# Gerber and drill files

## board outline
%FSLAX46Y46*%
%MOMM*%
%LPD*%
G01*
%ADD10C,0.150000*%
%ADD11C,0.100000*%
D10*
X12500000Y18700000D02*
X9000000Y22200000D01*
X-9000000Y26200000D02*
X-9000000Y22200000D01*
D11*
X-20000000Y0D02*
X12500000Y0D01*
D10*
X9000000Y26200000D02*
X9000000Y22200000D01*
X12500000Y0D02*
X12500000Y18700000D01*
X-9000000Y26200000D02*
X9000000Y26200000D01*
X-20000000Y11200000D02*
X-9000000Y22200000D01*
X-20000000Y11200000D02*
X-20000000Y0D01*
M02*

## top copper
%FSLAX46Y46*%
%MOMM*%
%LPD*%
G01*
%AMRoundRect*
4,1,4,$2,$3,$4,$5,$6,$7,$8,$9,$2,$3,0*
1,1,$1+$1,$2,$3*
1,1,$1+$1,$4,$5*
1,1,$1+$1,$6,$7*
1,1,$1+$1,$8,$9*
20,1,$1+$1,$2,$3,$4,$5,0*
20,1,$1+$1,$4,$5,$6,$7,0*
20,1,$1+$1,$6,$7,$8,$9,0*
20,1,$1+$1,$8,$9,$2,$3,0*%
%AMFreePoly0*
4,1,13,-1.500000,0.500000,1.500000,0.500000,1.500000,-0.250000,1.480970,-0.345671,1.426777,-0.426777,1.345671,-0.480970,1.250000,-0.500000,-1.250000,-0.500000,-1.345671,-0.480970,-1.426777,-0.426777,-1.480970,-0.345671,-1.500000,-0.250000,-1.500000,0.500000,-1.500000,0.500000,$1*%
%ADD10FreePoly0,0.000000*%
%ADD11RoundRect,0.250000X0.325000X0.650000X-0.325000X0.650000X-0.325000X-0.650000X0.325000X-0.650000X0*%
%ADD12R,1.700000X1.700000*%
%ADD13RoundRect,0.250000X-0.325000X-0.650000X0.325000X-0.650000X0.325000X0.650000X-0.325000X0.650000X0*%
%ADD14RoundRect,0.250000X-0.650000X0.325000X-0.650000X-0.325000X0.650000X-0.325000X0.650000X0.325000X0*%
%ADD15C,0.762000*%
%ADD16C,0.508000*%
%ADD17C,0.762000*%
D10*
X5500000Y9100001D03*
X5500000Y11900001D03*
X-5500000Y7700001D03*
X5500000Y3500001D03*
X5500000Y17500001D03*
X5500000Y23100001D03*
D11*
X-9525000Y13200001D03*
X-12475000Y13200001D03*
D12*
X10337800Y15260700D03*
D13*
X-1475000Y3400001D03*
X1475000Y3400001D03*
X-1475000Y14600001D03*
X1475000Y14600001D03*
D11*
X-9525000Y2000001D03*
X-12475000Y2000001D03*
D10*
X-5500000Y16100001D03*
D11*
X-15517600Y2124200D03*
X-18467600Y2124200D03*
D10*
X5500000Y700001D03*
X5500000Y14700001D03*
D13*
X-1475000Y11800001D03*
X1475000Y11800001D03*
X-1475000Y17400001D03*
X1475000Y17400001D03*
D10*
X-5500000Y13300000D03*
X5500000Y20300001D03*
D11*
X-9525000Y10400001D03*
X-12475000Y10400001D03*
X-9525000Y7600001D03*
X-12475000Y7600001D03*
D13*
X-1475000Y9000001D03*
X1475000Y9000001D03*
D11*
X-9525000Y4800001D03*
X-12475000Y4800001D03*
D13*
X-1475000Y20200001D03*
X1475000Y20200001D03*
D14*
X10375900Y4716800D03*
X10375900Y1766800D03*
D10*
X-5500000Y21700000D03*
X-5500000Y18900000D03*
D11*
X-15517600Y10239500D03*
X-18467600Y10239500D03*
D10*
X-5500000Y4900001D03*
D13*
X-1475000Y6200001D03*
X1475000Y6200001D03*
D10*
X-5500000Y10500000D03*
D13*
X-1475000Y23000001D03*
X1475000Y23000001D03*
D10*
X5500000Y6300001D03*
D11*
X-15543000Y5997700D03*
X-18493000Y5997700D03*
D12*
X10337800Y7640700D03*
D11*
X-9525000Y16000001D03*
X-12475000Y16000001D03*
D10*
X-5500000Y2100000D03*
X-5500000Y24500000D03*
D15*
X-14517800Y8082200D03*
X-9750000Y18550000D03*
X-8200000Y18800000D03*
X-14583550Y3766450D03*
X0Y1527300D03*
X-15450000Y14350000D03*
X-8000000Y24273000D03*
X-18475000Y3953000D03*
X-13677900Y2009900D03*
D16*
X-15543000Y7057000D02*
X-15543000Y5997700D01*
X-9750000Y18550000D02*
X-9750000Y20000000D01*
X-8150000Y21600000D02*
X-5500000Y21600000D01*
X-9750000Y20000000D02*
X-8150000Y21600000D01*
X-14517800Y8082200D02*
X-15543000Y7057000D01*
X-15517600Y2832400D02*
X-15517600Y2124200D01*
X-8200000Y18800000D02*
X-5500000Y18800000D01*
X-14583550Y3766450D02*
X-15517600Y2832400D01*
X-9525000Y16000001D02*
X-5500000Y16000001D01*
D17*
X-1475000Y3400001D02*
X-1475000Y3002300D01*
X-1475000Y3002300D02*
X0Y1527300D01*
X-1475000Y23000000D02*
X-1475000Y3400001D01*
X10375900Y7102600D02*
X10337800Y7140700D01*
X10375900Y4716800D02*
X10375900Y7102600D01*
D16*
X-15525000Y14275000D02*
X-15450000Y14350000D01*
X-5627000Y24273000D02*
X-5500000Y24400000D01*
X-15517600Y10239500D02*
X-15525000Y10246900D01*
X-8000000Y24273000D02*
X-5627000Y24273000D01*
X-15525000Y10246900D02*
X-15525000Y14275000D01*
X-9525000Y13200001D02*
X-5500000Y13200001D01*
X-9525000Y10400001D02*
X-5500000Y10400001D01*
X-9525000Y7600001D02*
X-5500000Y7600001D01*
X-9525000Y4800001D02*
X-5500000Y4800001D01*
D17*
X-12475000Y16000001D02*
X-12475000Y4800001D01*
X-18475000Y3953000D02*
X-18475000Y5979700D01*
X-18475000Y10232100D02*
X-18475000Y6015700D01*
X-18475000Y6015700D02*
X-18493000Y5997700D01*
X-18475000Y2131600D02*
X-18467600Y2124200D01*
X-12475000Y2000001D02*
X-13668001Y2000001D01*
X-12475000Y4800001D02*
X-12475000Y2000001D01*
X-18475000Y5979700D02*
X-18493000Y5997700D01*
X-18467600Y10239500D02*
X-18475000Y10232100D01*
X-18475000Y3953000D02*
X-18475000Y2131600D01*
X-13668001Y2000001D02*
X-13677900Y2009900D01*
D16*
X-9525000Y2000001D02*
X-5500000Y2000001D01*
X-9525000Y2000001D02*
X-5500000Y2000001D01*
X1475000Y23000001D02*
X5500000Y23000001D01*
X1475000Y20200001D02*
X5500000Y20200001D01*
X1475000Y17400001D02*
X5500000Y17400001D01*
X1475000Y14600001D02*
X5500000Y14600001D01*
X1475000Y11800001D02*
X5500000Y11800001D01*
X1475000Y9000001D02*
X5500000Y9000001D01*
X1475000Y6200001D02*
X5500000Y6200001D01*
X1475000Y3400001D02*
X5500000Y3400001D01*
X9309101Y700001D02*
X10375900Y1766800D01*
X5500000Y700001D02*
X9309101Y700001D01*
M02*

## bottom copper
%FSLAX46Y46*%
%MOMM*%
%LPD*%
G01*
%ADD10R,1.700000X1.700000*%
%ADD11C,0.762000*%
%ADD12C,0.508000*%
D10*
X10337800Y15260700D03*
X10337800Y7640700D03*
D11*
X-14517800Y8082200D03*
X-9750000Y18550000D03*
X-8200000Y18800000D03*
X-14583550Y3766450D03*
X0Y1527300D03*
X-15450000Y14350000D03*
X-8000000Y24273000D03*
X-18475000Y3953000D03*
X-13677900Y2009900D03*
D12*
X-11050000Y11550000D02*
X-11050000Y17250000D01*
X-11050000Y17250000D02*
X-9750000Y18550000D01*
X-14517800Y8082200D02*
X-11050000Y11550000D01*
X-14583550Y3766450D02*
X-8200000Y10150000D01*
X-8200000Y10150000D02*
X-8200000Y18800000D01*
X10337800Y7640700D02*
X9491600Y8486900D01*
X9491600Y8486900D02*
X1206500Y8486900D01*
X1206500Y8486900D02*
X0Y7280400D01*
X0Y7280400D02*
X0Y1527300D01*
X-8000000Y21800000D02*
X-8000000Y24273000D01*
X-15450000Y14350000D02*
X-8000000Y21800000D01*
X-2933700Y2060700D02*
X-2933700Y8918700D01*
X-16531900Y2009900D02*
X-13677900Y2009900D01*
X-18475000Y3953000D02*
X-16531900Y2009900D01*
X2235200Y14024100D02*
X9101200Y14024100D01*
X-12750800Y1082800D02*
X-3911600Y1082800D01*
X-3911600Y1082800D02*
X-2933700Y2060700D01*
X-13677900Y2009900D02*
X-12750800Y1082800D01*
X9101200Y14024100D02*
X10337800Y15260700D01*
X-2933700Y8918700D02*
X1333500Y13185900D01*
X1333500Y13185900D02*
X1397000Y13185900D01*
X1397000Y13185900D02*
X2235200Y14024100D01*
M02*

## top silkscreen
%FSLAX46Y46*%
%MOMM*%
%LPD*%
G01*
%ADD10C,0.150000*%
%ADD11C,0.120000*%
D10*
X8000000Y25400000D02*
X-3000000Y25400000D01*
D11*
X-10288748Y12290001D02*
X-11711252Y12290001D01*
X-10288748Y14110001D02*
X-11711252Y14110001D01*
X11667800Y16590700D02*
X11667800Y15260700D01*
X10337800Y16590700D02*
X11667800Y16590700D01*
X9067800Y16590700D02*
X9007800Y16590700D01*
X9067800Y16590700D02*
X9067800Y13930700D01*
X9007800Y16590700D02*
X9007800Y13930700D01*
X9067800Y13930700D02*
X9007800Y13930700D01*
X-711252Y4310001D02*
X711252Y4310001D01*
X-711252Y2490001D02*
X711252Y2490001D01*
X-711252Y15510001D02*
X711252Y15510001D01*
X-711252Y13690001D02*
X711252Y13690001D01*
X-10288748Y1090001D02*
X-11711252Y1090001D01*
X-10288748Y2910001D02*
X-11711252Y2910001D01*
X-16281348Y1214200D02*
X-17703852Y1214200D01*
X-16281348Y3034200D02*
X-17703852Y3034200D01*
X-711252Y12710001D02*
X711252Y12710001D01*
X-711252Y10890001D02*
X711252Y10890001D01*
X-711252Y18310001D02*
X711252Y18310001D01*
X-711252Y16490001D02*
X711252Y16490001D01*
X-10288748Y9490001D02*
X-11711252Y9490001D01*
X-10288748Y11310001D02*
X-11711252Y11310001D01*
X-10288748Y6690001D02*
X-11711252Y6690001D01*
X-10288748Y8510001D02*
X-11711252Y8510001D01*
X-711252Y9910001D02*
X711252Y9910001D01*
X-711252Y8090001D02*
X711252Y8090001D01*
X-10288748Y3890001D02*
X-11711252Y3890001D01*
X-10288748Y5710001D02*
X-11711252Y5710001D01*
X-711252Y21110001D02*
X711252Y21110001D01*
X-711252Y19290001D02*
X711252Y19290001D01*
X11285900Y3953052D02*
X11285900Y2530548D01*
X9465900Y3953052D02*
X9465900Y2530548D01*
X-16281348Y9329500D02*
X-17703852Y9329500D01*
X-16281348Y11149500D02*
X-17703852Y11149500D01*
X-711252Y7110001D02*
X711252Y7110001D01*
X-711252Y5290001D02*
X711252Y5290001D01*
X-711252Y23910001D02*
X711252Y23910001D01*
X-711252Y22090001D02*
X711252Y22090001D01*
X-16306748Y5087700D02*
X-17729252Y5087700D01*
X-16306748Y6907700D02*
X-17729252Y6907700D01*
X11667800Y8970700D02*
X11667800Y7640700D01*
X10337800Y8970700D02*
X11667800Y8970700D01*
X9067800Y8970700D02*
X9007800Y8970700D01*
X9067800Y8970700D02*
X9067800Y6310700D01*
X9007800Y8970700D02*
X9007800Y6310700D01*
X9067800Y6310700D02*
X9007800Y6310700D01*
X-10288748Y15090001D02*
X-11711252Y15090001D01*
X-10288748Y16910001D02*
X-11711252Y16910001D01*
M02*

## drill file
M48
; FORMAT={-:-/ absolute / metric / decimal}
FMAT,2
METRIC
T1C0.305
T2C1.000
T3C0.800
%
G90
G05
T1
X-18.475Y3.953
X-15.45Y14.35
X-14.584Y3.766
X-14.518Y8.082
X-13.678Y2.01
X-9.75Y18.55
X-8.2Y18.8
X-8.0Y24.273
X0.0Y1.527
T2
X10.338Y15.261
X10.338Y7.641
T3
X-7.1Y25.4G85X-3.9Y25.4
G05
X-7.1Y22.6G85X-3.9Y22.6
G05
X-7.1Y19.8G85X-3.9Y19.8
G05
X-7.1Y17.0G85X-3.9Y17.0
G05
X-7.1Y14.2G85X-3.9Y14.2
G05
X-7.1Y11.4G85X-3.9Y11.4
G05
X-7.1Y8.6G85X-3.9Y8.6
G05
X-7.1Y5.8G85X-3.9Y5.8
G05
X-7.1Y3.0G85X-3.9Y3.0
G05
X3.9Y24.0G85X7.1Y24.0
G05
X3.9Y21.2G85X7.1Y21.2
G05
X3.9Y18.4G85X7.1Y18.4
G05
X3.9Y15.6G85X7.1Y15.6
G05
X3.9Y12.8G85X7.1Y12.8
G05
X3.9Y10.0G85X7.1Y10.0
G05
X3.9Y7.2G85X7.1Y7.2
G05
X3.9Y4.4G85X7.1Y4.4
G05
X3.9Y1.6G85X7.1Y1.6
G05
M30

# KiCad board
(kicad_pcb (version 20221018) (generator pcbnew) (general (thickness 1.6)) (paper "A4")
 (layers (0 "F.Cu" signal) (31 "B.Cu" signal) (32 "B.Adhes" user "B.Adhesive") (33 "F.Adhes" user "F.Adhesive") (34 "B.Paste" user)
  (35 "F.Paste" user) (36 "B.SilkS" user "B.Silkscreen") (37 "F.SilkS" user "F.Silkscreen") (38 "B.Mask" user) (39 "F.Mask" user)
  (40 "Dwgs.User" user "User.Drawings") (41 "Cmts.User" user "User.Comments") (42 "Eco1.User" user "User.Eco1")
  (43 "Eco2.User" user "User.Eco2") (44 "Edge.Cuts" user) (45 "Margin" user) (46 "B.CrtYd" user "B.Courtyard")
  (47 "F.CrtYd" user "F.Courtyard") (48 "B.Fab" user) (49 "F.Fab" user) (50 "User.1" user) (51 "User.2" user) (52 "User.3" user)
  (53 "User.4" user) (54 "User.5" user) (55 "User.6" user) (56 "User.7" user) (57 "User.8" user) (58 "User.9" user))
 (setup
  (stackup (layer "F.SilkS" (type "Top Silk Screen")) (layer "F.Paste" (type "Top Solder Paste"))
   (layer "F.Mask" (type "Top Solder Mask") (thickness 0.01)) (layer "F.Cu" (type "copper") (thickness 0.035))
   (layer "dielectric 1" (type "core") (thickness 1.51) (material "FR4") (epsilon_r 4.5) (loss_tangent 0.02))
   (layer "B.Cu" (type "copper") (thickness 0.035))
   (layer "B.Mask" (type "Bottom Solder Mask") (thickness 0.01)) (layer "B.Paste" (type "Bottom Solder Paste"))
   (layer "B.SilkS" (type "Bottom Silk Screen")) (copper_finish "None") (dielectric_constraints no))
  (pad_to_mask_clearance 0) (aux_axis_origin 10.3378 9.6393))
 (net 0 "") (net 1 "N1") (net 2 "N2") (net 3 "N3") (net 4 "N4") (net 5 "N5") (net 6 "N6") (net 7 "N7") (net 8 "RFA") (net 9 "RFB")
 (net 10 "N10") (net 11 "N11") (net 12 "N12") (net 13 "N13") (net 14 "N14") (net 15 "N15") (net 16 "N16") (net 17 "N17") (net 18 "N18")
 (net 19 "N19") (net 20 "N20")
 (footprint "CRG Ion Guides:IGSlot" (layer "F.Cu") (at 5.5 -10.000001)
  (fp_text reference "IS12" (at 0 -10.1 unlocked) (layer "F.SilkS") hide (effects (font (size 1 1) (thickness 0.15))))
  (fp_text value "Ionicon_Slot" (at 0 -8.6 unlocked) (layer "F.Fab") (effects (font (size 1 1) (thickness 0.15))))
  (pad "" np_thru_hole oval (at 0 0) (size 4 0.8) (drill oval 4 0.8) (layers "*.Mask"))
  (pad "1" smd roundrect (at 0 0.9) (size 3 1) (layers "F.Cu" "F.Mask") (roundrect_rratio 0.25) (chamfer_ratio 0)
   (chamfer top_left top_right) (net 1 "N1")))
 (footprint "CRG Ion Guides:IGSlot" (layer "F.Cu") (at 5.5 -12.800001)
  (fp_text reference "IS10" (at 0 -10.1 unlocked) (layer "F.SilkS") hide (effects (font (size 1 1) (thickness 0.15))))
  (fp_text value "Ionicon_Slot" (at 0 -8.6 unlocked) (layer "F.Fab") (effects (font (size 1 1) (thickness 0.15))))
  (pad "" np_thru_hole oval (at 0 0) (size 4 0.8) (drill oval 4 0.8) (layers "*.Mask"))
  (pad "1" smd roundrect (at 0 0.9) (size 3 1) (layers "F.Cu" "F.Mask") (roundrect_rratio 0.25) (chamfer_ratio 0)
   (chamfer top_left top_right) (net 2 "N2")))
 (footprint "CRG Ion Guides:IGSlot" (layer "F.Cu") (at -5.5 -8.600001)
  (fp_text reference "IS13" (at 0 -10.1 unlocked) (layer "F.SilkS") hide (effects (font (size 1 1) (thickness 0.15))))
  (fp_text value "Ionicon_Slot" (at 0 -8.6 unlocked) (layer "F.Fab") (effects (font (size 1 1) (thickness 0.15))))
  (pad "" np_thru_hole oval (at 0 0) (size 4 0.8) (drill oval 4 0.8) (layers "*.Mask"))
  (pad "1" smd roundrect (at 0 0.9) (size 3 1) (layers "F.Cu" "F.Mask") (roundrect_rratio 0.25) (chamfer_ratio 0)
   (chamfer top_left top_right) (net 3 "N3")))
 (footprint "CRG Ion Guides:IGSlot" (layer "F.Cu") (at 5.5 -4.400001)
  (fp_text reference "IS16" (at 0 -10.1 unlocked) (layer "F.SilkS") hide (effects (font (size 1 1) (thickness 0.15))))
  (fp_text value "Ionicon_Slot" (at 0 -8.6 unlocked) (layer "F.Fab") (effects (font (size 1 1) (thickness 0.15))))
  (pad "" np_thru_hole oval (at 0 0) (size 4 0.8) (drill oval 4 0.8) (layers "*.Mask"))
  (pad "1" smd roundrect (at 0 0.9) (size 3 1) (layers "F.Cu" "F.Mask") (roundrect_rratio 0.25) (chamfer_ratio 0)
   (chamfer top_left top_right) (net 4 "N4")))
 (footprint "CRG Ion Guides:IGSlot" (layer "F.Cu") (at 5.5 -18.400001)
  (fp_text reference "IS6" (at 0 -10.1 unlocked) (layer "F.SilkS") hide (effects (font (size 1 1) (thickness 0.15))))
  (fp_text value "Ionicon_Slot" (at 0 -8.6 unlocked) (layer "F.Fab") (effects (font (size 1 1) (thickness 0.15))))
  (pad "" np_thru_hole oval (at 0 0) (size 4 0.8) (drill oval 4 0.8) (layers "*.Mask"))
  (pad "1" smd roundrect (at 0 0.9) (size 3 1) (layers "F.Cu" "F.Mask") (roundrect_rratio 0.25) (chamfer_ratio 0)
   (chamfer top_left top_right) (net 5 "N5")))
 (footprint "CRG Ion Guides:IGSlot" (layer "F.Cu") (at 5.5 -24.000001)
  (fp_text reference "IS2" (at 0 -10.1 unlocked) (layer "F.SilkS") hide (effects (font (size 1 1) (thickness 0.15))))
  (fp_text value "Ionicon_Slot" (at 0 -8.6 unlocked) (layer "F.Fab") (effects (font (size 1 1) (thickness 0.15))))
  (pad "" np_thru_hole oval (at 0 0) (size 4 0.8) (drill oval 4 0.8) (layers "*.Mask"))
  (pad "1" smd roundrect (at 0 0.9) (size 3 1) (layers "F.Cu" "F.Mask") (roundrect_rratio 0.25) (chamfer_ratio 0)
   (chamfer top_left top_right) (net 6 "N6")))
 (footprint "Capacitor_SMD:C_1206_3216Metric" (layer "F.Cu") (at -11 -13.200001 180)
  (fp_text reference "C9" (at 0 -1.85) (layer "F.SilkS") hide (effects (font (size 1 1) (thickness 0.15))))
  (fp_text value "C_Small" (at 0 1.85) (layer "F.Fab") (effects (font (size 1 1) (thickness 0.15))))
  (fp_line (start -0.711252 -0.91) (end 0.711252 -0.91) (stroke (width 0.12) (type solid)) (layer "F.SilkS"))
  (fp_line (start -0.711252 0.91) (end 0.711252 0.91) (stroke (width 0.12) (type solid)) (layer "F.SilkS"))
  (pad "1" smd roundrect (at -1.475 0 180) (size 1.15 1.8) (layers "F.Cu" "F.Paste" "F.Mask") (roundrect_rratio 0.2173913043) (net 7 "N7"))
  (pad "2" smd roundrect (at 1.475 0 180) (size 1.15 1.8) (layers "F.Cu" "F.Paste" "F.Mask") (roundrect_rratio 0.2173913043) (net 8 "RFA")))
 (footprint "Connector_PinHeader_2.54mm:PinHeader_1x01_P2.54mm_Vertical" (layer "F.Cu") (at 10.3378 -15.2607 -90)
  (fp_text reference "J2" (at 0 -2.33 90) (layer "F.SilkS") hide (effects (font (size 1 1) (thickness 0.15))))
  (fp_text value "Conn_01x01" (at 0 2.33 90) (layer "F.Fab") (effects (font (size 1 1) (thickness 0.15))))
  (fp_line (start -1.33 -1.33) (end 0 -1.33) (stroke (width 0.12) (type solid)) (layer "F.SilkS"))
  (fp_line (start -1.33 0) (end -1.33 -1.33) (stroke (width 0.12) (type solid)) (layer "F.SilkS"))
  (fp_line (start -1.33 1.27) (end -1.33 1.33) (stroke (width 0.12) (type solid)) (layer "F.SilkS"))
  (fp_line (start -1.33 1.27) (end 1.33 1.27) (stroke (width 0.12) (type solid)) (layer "F.SilkS"))
  (fp_line (start -1.33 1.33) (end 1.33 1.33) (stroke (width 0.12) (type solid)) (layer "F.SilkS"))
  (fp_line (start 1.33 1.27) (end 1.33 1.33) (stroke (width 0.12) (type solid)) (layer "F.SilkS"))
  (pad "1" thru_hole rect (at 0 0 270) (size 1.7 1.7) (drill 1) (layers "*.Cu" "*.Mask") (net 8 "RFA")))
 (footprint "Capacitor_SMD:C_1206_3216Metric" (layer "F.Cu") (at 0 -3.400001)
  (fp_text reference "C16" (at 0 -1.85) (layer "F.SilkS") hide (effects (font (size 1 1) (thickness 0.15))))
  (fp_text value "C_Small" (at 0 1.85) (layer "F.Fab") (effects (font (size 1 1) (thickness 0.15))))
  (fp_line (start -0.711252 -0.91) (end 0.711252 -0.91) (stroke (width 0.12) (type solid)) (layer "F.SilkS"))
  (fp_line (start -0.711252 0.91) (end 0.711252 0.91) (stroke (width 0.12) (type solid)) (layer "F.SilkS"))
  (pad "1" smd roundrect (at -1.475 0) (size 1.15 1.8) (layers "F.Cu" "F.Paste" "F.Mask") (roundrect_rratio 0.2173913043) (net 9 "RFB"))
  (pad "2" smd roundrect (at 1.475 0) (size 1.15 1.8) (layers "F.Cu" "F.Paste" "F.Mask") (roundrect_rratio 0.2173913043) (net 4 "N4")))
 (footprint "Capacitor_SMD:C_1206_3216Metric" (layer "F.Cu") (at 0 -14.600001)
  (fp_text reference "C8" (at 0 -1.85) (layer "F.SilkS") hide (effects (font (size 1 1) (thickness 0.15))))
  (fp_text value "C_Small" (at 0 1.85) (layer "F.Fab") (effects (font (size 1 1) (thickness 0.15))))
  (fp_line (start -0.711252 -0.91) (end 0.711252 -0.91) (stroke (width 0.12) (type solid)) (layer "F.SilkS"))
  (fp_line (start -0.711252 0.91) (end 0.711252 0.91) (stroke (width 0.12) (type solid)) (layer "F.SilkS"))
  (pad "1" smd roundrect (at -1.475 0) (size 1.15 1.8) (layers "F.Cu" "F.Paste" "F.Mask") (roundrect_rratio 0.2173913043) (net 9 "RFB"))
  (pad "2" smd roundrect (at 1.475 0) (size 1.15 1.8) (layers "F.Cu" "F.Paste" "F.Mask") (roundrect_rratio 0.2173913043) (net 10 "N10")))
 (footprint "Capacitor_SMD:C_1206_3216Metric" (layer "F.Cu") (at -11 -2.000001 180)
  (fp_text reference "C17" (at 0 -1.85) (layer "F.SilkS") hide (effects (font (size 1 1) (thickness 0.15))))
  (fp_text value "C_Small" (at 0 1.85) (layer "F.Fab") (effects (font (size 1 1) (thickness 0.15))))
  (fp_line (start -0.711252 -0.91) (end 0.711252 -0.91) (stroke (width 0.12) (type solid)) (layer "F.SilkS"))
  (fp_line (start -0.711252 0.91) (end 0.711252 0.91) (stroke (width 0.12) (type solid)) (layer "F.SilkS"))
  (pad "1" smd roundrect (at -1.475 0 180) (size 1.15 1.8) (layers "F.Cu" "F.Paste" "F.Mask") (roundrect_rratio 0.2173913043) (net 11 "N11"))
  (pad "2" smd roundrect (at 1.475 0 180) (size 1.15 1.8) (layers "F.Cu" "F.Paste" "F.Mask") (roundrect_rratio 0.2173913043) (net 8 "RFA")))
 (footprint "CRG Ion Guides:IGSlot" (layer "F.Cu") (at -5.5 -17.000001)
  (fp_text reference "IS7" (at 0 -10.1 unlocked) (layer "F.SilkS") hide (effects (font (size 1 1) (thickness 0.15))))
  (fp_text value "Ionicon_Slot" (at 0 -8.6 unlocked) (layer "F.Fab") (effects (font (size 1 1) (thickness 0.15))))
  (pad "" np_thru_hole oval (at 0 0) (size 4 0.8) (drill oval 4 0.8) (layers "*.Mask"))
  (pad "1" smd roundrect (at 0 0.9) (size 3 1) (layers "F.Cu" "F.Mask") (roundrect_rratio 0.25) (chamfer_ratio 0)
   (chamfer top_left top_right) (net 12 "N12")))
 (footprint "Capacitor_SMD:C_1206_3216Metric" (layer "F.Cu") (at -16.9926 -2.1242 180)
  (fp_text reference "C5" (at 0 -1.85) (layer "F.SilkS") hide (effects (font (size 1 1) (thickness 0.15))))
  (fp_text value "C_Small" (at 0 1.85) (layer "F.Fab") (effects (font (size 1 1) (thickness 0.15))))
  (fp_line (start -0.711252 -0.91) (end 0.711252 -0.91) (stroke (width 0.12) (type solid)) (layer "F.SilkS"))
  (fp_line (start -0.711252 0.91) (end 0.711252 0.91) (stroke (width 0.12) (type solid)) (layer "F.SilkS"))
  (pad "1" smd roundrect (at -1.475 0 180) (size 1.15 1.8) (layers "F.Cu" "F.Paste" "F.Mask") (roundrect_rratio 0.2173913043) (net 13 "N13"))
  (pad "2" smd roundrect (at 1.475 0 180) (size 1.15 1.8) (layers "F.Cu" "F.Paste" "F.Mask") (roundrect_rratio 0.2173913043) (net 8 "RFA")))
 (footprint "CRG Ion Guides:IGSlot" (layer "F.Cu") (at 5.5 -1.600001)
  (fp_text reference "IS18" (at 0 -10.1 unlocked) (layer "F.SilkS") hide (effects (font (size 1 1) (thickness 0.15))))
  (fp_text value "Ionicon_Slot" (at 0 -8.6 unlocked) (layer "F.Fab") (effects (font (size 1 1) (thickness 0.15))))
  (pad "" np_thru_hole oval (at 0 0) (size 4 0.8) (drill oval 4 0.8) (layers "*.Mask"))
  (pad "1" smd roundrect (at 0 0.9) (size 3 1) (layers "F.Cu" "F.Mask") (roundrect_rratio 0.25) (chamfer_ratio 0)
   (chamfer top_left top_right) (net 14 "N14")))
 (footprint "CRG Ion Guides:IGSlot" (layer "F.Cu") (at 5.5 -15.600001)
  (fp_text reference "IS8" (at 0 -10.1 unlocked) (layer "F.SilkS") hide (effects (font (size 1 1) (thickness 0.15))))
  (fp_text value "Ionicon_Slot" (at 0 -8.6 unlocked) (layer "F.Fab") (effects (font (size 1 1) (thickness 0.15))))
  (pad "" np_thru_hole oval (at 0 0) (size 4 0.8) (drill oval 4 0.8) (layers "*.Mask"))
  (pad "1" smd roundrect (at 0 0.9) (size 3 1) (layers "F.Cu" "F.Mask") (roundrect_rratio 0.25) (chamfer_ratio 0)
   (chamfer top_left top_right) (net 10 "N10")))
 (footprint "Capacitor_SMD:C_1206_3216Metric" (layer "F.Cu") (at 0 -11.800001)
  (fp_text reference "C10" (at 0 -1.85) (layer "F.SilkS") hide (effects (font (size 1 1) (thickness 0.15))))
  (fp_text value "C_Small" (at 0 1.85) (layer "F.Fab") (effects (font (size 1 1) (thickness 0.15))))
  (fp_line (start -0.711252 -0.91) (end 0.711252 -0.91) (stroke (width 0.12) (type solid)) (layer "F.SilkS"))
  (fp_line (start -0.711252 0.91) (end 0.711252 0.91) (stroke (width 0.12) (type solid)) (layer "F.SilkS"))
  (pad "1" smd roundrect (at -1.475 0) (size 1.15 1.8) (layers "F.Cu" "F.Paste" "F.Mask") (roundrect_rratio 0.2173913043) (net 9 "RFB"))
  (pad "2" smd roundrect (at 1.475 0) (size 1.15 1.8) (layers "F.Cu" "F.Paste" "F.Mask") (roundrect_rratio 0.2173913043) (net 2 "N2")))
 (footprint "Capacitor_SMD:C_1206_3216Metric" (layer "F.Cu") (at 0 -17.400001)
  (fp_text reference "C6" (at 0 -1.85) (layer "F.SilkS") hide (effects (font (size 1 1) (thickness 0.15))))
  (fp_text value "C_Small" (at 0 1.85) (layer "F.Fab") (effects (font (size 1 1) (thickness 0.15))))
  (fp_line (start -0.711252 -0.91) (end 0.711252 -0.91) (stroke (width 0.12) (type solid)) (layer "F.SilkS"))
  (fp_line (start -0.711252 0.91) (end 0.711252 0.91) (stroke (width 0.12) (type solid)) (layer "F.SilkS"))
  (pad "1" smd roundrect (at -1.475 0) (size 1.15 1.8) (layers "F.Cu" "F.Paste" "F.Mask") (roundrect_rratio 0.2173913043) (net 9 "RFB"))
  (pad "2" smd roundrect (at 1.475 0) (size 1.15 1.8) (layers "F.Cu" "F.Paste" "F.Mask") (roundrect_rratio 0.2173913043) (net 5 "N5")))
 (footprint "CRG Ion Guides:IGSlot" (layer "F.Cu") (at -5.5 -14.2)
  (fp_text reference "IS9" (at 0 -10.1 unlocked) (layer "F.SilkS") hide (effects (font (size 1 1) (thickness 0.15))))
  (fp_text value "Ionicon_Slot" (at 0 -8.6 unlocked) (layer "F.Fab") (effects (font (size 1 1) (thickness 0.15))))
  (pad "" np_thru_hole oval (at 0 0) (size 4 0.8) (drill oval 4 0.8) (layers "*.Mask"))
  (pad "1" smd roundrect (at 0 0.9) (size 3 1) (layers "F.Cu" "F.Mask") (roundrect_rratio 0.25) (chamfer_ratio 0)
   (chamfer top_left top_right) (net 7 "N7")))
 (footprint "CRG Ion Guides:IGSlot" (layer "F.Cu") (at 5.5 -21.200001)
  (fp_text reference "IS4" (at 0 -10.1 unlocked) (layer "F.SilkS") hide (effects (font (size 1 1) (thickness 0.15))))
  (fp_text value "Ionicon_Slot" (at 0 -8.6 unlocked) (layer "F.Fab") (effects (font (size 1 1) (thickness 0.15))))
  (pad "" np_thru_hole oval (at 0 0) (size 4 0.8) (drill oval 4 0.8) (layers "*.Mask"))
  (pad "1" smd roundrect (at 0 0.9) (size 3 1) (layers "F.Cu" "F.Mask") (roundrect_rratio 0.25) (chamfer_ratio 0)
   (chamfer top_left top_right) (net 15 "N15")))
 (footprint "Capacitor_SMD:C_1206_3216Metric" (layer "F.Cu") (at -11 -10.400001 180)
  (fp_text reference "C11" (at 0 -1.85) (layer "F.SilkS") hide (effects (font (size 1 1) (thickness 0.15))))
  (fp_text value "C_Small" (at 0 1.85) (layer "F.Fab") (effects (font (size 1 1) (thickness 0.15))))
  (fp_line (start -0.711252 -0.91) (end 0.711252 -0.91) (stroke (width 0.12) (type solid)) (layer "F.SilkS"))
  (fp_line (start -0.711252 0.91) (end 0.711252 0.91) (stroke (width 0.12) (type solid)) (layer "F.SilkS"))
  (pad "1" smd roundrect (at -1.475 0 180) (size 1.15 1.8) (layers "F.Cu" "F.Paste" "F.Mask") (roundrect_rratio 0.2173913043) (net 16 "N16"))
  (pad "2" smd roundrect (at 1.475 0 180) (size 1.15 1.8) (layers "F.Cu" "F.Paste" "F.Mask") (roundrect_rratio 0.2173913043) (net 8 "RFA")))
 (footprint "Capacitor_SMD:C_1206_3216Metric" (layer "F.Cu") (at -11 -7.600001 180)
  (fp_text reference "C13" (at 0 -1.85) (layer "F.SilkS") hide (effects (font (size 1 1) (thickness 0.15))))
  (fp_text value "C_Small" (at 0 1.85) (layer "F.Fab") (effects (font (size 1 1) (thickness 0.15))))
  (fp_line (start -0.711252 -0.91) (end 0.711252 -0.91) (stroke (width 0.12) (type solid)) (layer "F.SilkS"))
  (fp_line (start -0.711252 0.91) (end 0.711252 0.91) (stroke (width 0.12) (type solid)) (layer "F.SilkS"))
  (pad "1" smd roundrect (at -1.475 0 180) (size 1.15 1.8) (layers "F.Cu" "F.Paste" "F.Mask") (roundrect_rratio 0.2173913043) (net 3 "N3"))
  (pad "2" smd roundrect (at 1.475 0 180) (size 1.15 1.8) (layers "F.Cu" "F.Paste" "F.Mask") (roundrect_rratio 0.2173913043) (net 8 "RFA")))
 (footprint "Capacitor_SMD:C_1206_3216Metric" (layer "F.Cu") (at 0 -9.000001)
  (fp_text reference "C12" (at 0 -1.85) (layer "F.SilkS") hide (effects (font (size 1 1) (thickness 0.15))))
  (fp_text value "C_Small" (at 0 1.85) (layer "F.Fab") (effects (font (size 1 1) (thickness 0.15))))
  (fp_line (start -0.711252 -0.91) (end 0.711252 -0.91) (stroke (width 0.12) (type solid)) (layer "F.SilkS"))
  (fp_line (start -0.711252 0.91) (end 0.711252 0.91) (stroke (width 0.12) (type solid)) (layer "F.SilkS"))
  (pad "1" smd roundrect (at -1.475 0) (size 1.15 1.8) (layers "F.Cu" "F.Paste" "F.Mask") (roundrect_rratio 0.2173913043) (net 9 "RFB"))
  (pad "2" smd roundrect (at 1.475 0) (size 1.15 1.8) (layers "F.Cu" "F.Paste" "F.Mask") (roundrect_rratio 0.2173913043) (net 1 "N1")))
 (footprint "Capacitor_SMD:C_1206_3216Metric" (layer "F.Cu") (at -11 -4.800001 180)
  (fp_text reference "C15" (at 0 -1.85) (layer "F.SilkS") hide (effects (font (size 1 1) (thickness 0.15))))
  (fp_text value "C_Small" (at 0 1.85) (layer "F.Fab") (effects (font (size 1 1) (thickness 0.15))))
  (fp_line (start -0.711252 -0.91) (end 0.711252 -0.91) (stroke (width 0.12) (type solid)) (layer "F.SilkS"))
  (fp_line (start -0.711252 0.91) (end 0.711252 0.91) (stroke (width 0.12) (type solid)) (layer "F.SilkS"))
  (pad "1" smd roundrect (at -1.475 0 180) (size 1.15 1.8) (layers "F.Cu" "F.Paste" "F.Mask") (roundrect_rratio 0.2173913043) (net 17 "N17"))
  (pad "2" smd roundrect (at 1.475 0 180) (size 1.15 1.8) (layers "F.Cu" "F.Paste" "F.Mask") (roundrect_rratio 0.2173913043) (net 8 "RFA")))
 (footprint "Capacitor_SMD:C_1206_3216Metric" (layer "F.Cu") (at 0 -20.200001)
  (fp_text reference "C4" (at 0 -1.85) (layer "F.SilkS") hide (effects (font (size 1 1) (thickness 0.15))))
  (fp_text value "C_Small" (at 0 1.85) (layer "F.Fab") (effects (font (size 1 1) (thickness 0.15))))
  (fp_line (start -0.711252 -0.91) (end 0.711252 -0.91) (stroke (width 0.12) (type solid)) (layer "F.SilkS"))
  (fp_line (start -0.711252 0.91) (end 0.711252 0.91) (stroke (width 0.12) (type solid)) (layer "F.SilkS"))
  (pad "1" smd roundrect (at -1.475 0) (size 1.15 1.8) (layers "F.Cu" "F.Paste" "F.Mask") (roundrect_rratio 0.2173913043) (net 9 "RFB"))
  (pad "2" smd roundrect (at 1.475 0) (size 1.15 1.8) (layers "F.Cu" "F.Paste" "F.Mask") (roundrect_rratio 0.2173913043) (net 15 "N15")))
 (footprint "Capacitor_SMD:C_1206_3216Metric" (layer "F.Cu") (at 10.3759 -3.2418 -90)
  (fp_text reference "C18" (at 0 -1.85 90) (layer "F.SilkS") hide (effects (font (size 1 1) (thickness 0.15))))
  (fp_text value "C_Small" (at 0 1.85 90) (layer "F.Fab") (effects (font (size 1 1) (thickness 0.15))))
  (fp_line (start -0.711252 -0.91) (end 0.711252 -0.91) (stroke (width 0.12) (type solid)) (layer "F.SilkS"))
  (fp_line (start -0.711252 0.91) (end 0.711252 0.91) (stroke (width 0.12) (type solid)) (layer "F.SilkS"))
  (pad "1" smd roundrect (at -1.475 0 270) (size 1.15 1.8) (layers "F.Cu" "F.Paste" "F.Mask") (roundrect_rratio 0.2173913043) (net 9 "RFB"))
  (pad "2" smd roundrect (at 1.475 0 270) (size 1.15 1.8) (layers "F.Cu" "F.Paste" "F.Mask") (roundrect_rratio 0.2173913043) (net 14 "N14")))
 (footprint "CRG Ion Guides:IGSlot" (layer "F.Cu") (at -5.5 -22.6)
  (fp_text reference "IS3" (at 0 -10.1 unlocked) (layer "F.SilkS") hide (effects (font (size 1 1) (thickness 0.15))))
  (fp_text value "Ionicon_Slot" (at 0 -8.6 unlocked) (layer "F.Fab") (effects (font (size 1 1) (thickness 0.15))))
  (pad "" np_thru_hole oval (at 0 0) (size 4 0.8) (drill oval 4 0.8) (layers "*.Mask"))
  (pad "1" smd roundrect (at 0 0.9) (size 3 1) (layers "F.Cu" "F.Mask") (roundrect_rratio 0.25) (chamfer_ratio 0)
   (chamfer top_left top_right) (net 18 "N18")))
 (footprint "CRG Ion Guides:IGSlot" (layer "F.Cu") (at -5.5 -19.8)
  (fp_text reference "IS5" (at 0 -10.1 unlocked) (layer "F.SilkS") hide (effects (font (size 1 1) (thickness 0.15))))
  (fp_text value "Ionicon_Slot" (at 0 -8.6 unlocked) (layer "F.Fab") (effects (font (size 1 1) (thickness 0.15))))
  (pad "" np_thru_hole oval (at 0 0) (size 4 0.8) (drill oval 4 0.8) (layers "*.Mask"))
  (pad "1" smd roundrect (at 0 0.9) (size 3 1) (layers "F.Cu" "F.Mask") (roundrect_rratio 0.25) (chamfer_ratio 0)
   (chamfer top_left top_right) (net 13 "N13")))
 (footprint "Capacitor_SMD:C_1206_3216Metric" (layer "F.Cu") (at -16.9926 -10.2395 180)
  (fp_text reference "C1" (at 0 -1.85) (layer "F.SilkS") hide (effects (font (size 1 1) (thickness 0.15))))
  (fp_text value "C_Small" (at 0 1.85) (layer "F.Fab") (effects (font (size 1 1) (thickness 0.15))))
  (fp_line (start -0.711252 -0.91) (end 0.711252 -0.91) (stroke (width 0.12) (type solid)) (layer "F.SilkS"))
  (fp_line (start -0.711252 0.91) (end 0.711252 0.91) (stroke (width 0.12) (type solid)) (layer "F.SilkS"))
  (pad "1" smd roundrect (at -1.475 0 180) (size 1.15 1.8) (layers "F.Cu" "F.Paste" "F.Mask") (roundrect_rratio 0.2173913043) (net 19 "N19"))
  (pad "2" smd roundrect (at 1.475 0 180) (size 1.15 1.8) (layers "F.Cu" "F.Paste" "F.Mask") (roundrect_rratio 0.2173913043) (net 8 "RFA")))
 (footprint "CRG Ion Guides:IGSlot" (layer "F.Cu") (at -5.5 -5.800001)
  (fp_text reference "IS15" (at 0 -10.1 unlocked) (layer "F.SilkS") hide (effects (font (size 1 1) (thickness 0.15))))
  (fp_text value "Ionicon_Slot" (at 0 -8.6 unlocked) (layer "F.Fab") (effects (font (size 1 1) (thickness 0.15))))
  (pad "" np_thru_hole oval (at 0 0) (size 4 0.8) (drill oval 4 0.8) (layers "*.Mask"))
  (pad "1" smd roundrect (at 0 0.9) (size 3 1) (layers "F.Cu" "F.Mask") (roundrect_rratio 0.25) (chamfer_ratio 0)
   (chamfer top_left top_right) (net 17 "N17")))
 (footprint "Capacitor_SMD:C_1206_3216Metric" (layer "F.Cu") (at 0 -6.200001)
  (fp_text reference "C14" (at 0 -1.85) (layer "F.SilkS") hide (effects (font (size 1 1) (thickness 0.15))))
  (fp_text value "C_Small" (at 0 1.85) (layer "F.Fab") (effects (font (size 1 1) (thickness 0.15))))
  (fp_line (start -0.711252 -0.91) (end 0.711252 -0.91) (stroke (width 0.12) (type solid)) (layer "F.SilkS"))
  (fp_line (start -0.711252 0.91) (end 0.711252 0.91) (stroke (width 0.12) (type solid)) (layer "F.SilkS"))
  (pad "1" smd roundrect (at -1.475 0) (size 1.15 1.8) (layers "F.Cu" "F.Paste" "F.Mask") (roundrect_rratio 0.2173913043) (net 9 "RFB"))
  (pad "2" smd roundrect (at 1.475 0) (size 1.15 1.8) (layers "F.Cu" "F.Paste" "F.Mask") (roundrect_rratio 0.2173913043) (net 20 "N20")))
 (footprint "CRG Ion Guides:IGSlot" (layer "F.Cu") (at -5.5 -11.4)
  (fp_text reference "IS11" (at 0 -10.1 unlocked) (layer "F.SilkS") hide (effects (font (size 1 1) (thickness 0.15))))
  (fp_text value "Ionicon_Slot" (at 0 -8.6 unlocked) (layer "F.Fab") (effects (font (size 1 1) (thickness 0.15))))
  (pad "" np_thru_hole oval (at 0 0) (size 4 0.8) (drill oval 4 0.8) (layers "*.Mask"))
  (pad "1" smd roundrect (at 0 0.9) (size 3 1) (layers "F.Cu" "F.Mask") (roundrect_rratio 0.25) (chamfer_ratio 0)
   (chamfer top_left top_right) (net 16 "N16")))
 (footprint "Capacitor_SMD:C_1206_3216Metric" (layer "F.Cu") (at 0 -23.000001)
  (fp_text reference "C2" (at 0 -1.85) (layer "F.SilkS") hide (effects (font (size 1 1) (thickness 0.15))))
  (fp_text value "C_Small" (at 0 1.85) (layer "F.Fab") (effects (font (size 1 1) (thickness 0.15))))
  (fp_line (start -0.711252 -0.91) (end 0.711252 -0.91) (stroke (width 0.12) (type solid)) (layer "F.SilkS"))
  (fp_line (start -0.711252 0.91) (end 0.711252 0.91) (stroke (width 0.12) (type solid)) (layer "F.SilkS"))
  (pad "1" smd roundrect (at -1.475 0) (size 1.15 1.8) (layers "F.Cu" "F.Paste" "F.Mask") (roundrect_rratio 0.2173913043) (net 9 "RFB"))
  (pad "2" smd roundrect (at 1.475 0) (size 1.15 1.8) (layers "F.Cu" "F.Paste" "F.Mask") (roundrect_rratio 0.2173913043) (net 6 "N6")))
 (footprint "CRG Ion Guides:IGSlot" (layer "F.Cu") (at 5.5 -7.200001)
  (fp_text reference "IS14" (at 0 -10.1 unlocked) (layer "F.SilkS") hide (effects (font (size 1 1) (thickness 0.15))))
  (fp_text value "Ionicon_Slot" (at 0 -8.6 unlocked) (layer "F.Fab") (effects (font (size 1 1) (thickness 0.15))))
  (pad "" np_thru_hole oval (at 0 0) (size 4 0.8) (drill oval 4 0.8) (layers "*.Mask"))
  (pad "1" smd roundrect (at 0 0.9) (size 3 1) (layers "F.Cu" "F.Mask") (roundrect_rratio 0.25) (chamfer_ratio 0)
   (chamfer top_left top_right) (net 20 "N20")))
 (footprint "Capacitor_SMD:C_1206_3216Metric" (layer "F.Cu") (at -17.018 -5.9977 180)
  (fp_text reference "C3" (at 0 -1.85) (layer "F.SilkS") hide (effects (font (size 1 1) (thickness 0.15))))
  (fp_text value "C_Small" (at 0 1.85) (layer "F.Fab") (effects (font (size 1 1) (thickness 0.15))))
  (fp_line (start -0.711252 -0.91) (end 0.711252 -0.91) (stroke (width 0.12) (type solid)) (layer "F.SilkS"))
  (fp_line (start -0.711252 0.91) (end 0.711252 0.91) (stroke (width 0.12) (type solid)) (layer "F.SilkS"))
  (pad "1" smd roundrect (at -1.475 0 180) (size 1.15 1.8) (layers "F.Cu" "F.Paste" "F.Mask") (roundrect_rratio 0.2173913043) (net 18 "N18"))
  (pad "2" smd roundrect (at 1.475 0 180) (size 1.15 1.8) (layers "F.Cu" "F.Paste" "F.Mask") (roundrect_rratio 0.2173913043) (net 8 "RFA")))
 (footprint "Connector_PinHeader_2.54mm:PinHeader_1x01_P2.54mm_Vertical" (layer "F.Cu") (at 10.3378 -7.6407 -90)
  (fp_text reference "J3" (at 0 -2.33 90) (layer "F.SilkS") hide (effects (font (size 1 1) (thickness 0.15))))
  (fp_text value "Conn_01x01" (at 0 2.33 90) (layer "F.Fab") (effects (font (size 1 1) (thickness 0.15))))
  (fp_line (start -1.33 -1.33) (end 0 -1.33) (stroke (width 0.12) (type solid)) (layer "F.SilkS"))
  (fp_line (start -1.33 0) (end -1.33 -1.33) (stroke (width 0.12) (type solid)) (layer "F.SilkS"))
  (fp_line (start -1.33 1.27) (end -1.33 1.33) (stroke (width 0.12) (type solid)) (layer "F.SilkS"))
  (fp_line (start -1.33 1.27) (end 1.33 1.27) (stroke (width 0.12) (type solid)) (layer "F.SilkS"))
  (fp_line (start -1.33 1.33) (end 1.33 1.33) (stroke (width 0.12) (type solid)) (layer "F.SilkS"))
  (fp_line (start 1.33 1.27) (end 1.33 1.33) (stroke (width 0.12) (type solid)) (layer "F.SilkS"))
  (pad "1" thru_hole rect (at 0 0 270) (size 1.7 1.7) (drill 1) (layers "*.Cu" "*.Mask") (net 9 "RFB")))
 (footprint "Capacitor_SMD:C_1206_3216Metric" (layer "F.Cu") (at -11 -16.000001 180)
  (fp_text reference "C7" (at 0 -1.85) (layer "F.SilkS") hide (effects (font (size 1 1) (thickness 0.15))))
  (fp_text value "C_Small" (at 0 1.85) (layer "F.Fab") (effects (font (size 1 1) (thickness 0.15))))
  (fp_line (start -0.711252 -0.91) (end 0.711252 -0.91) (stroke (width 0.12) (type solid)) (layer "F.SilkS"))
  (fp_line (start -0.711252 0.91) (end 0.711252 0.91) (stroke (width 0.12) (type solid)) (layer "F.SilkS"))
  (pad "1" smd roundrect (at -1.475 0 180) (size 1.15 1.8) (layers "F.Cu" "F.Paste" "F.Mask") (roundrect_rratio 0.2173913043) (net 12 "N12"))
  (pad "2" smd roundrect (at 1.475 0 180) (size 1.15 1.8) (layers "F.Cu" "F.Paste" "F.Mask") (roundrect_rratio 0.2173913043) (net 8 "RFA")))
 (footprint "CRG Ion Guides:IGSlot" (layer "F.Cu") (at -5.5 -3)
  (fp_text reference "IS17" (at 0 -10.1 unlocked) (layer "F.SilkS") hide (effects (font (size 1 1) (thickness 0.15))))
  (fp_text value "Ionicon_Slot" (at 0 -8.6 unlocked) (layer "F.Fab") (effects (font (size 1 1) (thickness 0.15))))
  (pad "" np_thru_hole oval (at 0 0) (size 4 0.8) (drill oval 4 0.8) (layers "*.Mask"))
  (pad "1" smd roundrect (at 0 0.9) (size 3 1) (layers "F.Cu" "F.Mask") (roundrect_rratio 0.25) (chamfer_ratio 0)
   (chamfer top_left top_right) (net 11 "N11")))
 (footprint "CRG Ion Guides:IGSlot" (layer "F.Cu") (at -5.5 -25.4)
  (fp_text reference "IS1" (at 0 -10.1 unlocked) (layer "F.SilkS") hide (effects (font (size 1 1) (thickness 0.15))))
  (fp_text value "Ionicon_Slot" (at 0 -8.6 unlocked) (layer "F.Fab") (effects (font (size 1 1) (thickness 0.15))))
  (pad "" np_thru_hole oval (at 0 0) (size 4 0.8) (drill oval 4 0.8) (layers "*.Mask"))
  (pad "1" smd roundrect (at 0 0.9) (size 3 1) (layers "F.Cu" "F.Mask") (roundrect_rratio 0.25) (chamfer_ratio 0)
   (chamfer top_left top_right) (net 19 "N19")))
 (gr_line (start 8 -25.4) (end -3 -25.4) (stroke (width 0.15) (type solid)) (layer "F.SilkS"))
 (gr_line (start 12.5 -18.7) (end 9 -22.2) (stroke (width 0.15) (type solid)) (layer "Edge.Cuts"))
 (gr_line (start -9 -26.2) (end -9 -22.2) (stroke (width 0.15) (type solid)) (layer "Edge.Cuts"))
 (gr_line (start -20 0) (end 12.5 0) (stroke (width 0.1) (type solid)) (layer "Edge.Cuts"))
 (gr_line (start 9 -26.2) (end 9 -22.2) (stroke (width 0.15) (type solid)) (layer "Edge.Cuts"))
 (gr_line (start 12.5 0) (end 12.5 -18.7) (stroke (width 0.15) (type solid)) (layer "Edge.Cuts"))
 (gr_line (start -9 -26.2) (end 9 -26.2) (stroke (width 0.15) (type solid)) (layer "Edge.Cuts"))
 (gr_line (start -20 -11.2) (end -9 -22.2) (stroke (width 0.15) (type solid)) (layer "Edge.Cuts"))
 (gr_line (start -20 -11.2) (end -20 0) (stroke (width 0.15) (type solid)) (layer "Edge.Cuts"))
 (segment (start -15.543 -7.057) (end -15.543 -5.9977) (width 0.508) (layer "F.Cu") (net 18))
 (segment (start -9.75 -18.55) (end -9.75 -20) (width 0.508) (layer "F.Cu") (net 18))
 (segment (start -8.15 -21.6) (end -5.5 -21.6) (width 0.508) (layer "F.Cu") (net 18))
 (segment (start -9.75 -20) (end -8.15 -21.6) (width 0.508) (layer "F.Cu") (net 18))
 (segment (start -14.5178 -8.0822) (end -15.543 -7.057) (width 0.508) (layer "F.Cu") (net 18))
 (via (at -14.5178 -8.0822) (size 0.762) (drill 0.3048) (layers "F.Cu" "B.Cu") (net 18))
 (via (at -9.75 -18.55) (size 0.762) (drill 0.3048) (layers "F.Cu" "B.Cu") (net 18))
 (segment (start -11.05 -11.55) (end -11.05 -17.25) (width 0.508) (layer "B.Cu") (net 18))
 (segment (start -11.05 -17.25) (end -9.75 -18.55) (width 0.508) (layer "B.Cu") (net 18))
 (segment (start -14.5178 -8.0822) (end -11.05 -11.55) (width 0.508) (layer "B.Cu") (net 18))
 (segment (start -15.5176 -2.8324) (end -15.5176 -2.1242) (width 0.508) (layer "F.Cu") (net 13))
 (segment (start -8.2 -18.8) (end -5.5 -18.8) (width 0.508) (layer "F.Cu") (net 13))
 (segment (start -14.58355 -3.76645) (end -15.5176 -2.8324) (width 0.508) (layer "F.Cu") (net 13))
 (via (at -8.2 -18.8) (size 0.762) (drill 0.3048) (layers "F.Cu" "B.Cu") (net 13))
 (via (at -14.58355 -3.76645) (size 0.762) (drill 0.3048) (layers "F.Cu" "B.Cu") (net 13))
 (segment (start -14.58355 -3.76645) (end -8.2 -10.15) (width 0.508) (layer "B.Cu") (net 13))
 (segment (start -8.2 -10.15) (end -8.2 -18.8) (width 0.508) (layer "B.Cu") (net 13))
 (segment (start -9.525 -16.000001) (end -5.5 -16.000001) (width 0.508) (layer "F.Cu") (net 12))
 (segment (start -1.475 -3.400001) (end -1.475 -3.0023) (width 0.762) (layer "F.Cu") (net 9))
 (segment (start -1.475 -3.0023) (end 0 -1.5273) (width 0.762) (layer "F.Cu") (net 9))
 (segment (start -1.475 -23) (end -1.475 -3.400001) (width 0.762) (layer "F.Cu") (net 9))
 (segment (start 10.3759 -7.1026) (end 10.3378 -7.1407) (width 0.762) (layer "F.Cu") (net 9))
 (segment (start 10.3759 -4.7168) (end 10.3759 -7.1026) (width 0.762) (layer "F.Cu") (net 9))
 (via (at 0 -1.5273) (size 0.762) (drill 0.3048) (layers "F.Cu" "B.Cu") (free) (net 9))
 (segment (start 10.3378 -7.6407) (end 9.4916 -8.4869) (width 0.508) (layer "B.Cu") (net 9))
 (segment (start 9.4916 -8.4869) (end 1.2065 -8.4869) (width 0.508) (layer "B.Cu") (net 9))
 (segment (start 1.2065 -8.4869) (end 0 -7.2804) (width 0.508) (layer "B.Cu") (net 9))
 (segment (start 0 -7.2804) (end 0 -1.5273) (width 0.508) (layer "B.Cu") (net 9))
 (segment (start -15.525 -14.275) (end -15.45 -14.35) (width 0.508) (layer "F.Cu") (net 19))
 (segment (start -5.627 -24.273) (end -5.5 -24.4) (width 0.508) (layer "F.Cu") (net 19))
 (segment (start -15.5176 -10.2395) (end -15.525 -10.2469) (width 0.508) (layer "F.Cu") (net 19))
 (segment (start -8 -24.273) (end -5.627 -24.273) (width 0.508) (layer "F.Cu") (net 19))
 (segment (start -15.525 -10.2469) (end -15.525 -14.275) (width 0.508) (layer "F.Cu") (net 19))
 (via (at -15.45 -14.35) (size 0.762) (drill 0.3048) (layers "F.Cu" "B.Cu") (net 19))
 (via (at -8 -24.273) (size 0.762) (drill 0.3048) (layers "F.Cu" "B.Cu") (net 19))
 (segment (start -8 -21.8) (end -8 -24.273) (width 0.508) (layer "B.Cu") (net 19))
 (segment (start -15.45 -14.35) (end -8 -21.8) (width 0.508) (layer "B.Cu") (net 19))
 (segment (start -9.525 -13.200001) (end -5.5 -13.200001) (width 0.508) (layer "F.Cu") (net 7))
 (segment (start -9.525 -10.400001) (end -5.5 -10.400001) (width 0.508) (layer "F.Cu") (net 16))
 (segment (start -9.525 -7.600001) (end -5.5 -7.600001) (width 0.508) (layer "F.Cu") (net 3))
 (segment (start -9.525 -4.800001) (end -5.5 -4.800001) (width 0.508) (layer "F.Cu") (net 17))
 (segment (start -12.475 -16.000001) (end -12.475 -4.800001) (width 0.762) (layer "F.Cu") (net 8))
 (segment (start -18.475 -3.953) (end -18.475 -5.9797) (width 0.762) (layer "F.Cu") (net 8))
 (segment (start -18.475 -10.2321) (end -18.475 -6.0157) (width 0.762) (layer "F.Cu") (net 8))
 (segment (start -18.475 -6.0157) (end -18.493 -5.9977) (width 0.762) (layer "F.Cu") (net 8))
 (segment (start -18.475 -2.1316) (end -18.4676 -2.1242) (width 0.762) (layer "F.Cu") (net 8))
 (segment (start -12.475 -2.000001) (end -13.668001 -2.000001) (width 0.762) (layer "F.Cu") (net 8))
 (segment (start -12.475 -4.800001) (end -12.475 -2.000001) (width 0.762) (layer "F.Cu") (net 8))
 (segment (start -18.475 -5.9797) (end -18.493 -5.9977) (width 0.762) (layer "F.Cu") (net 8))
 (segment (start -18.4676 -10.2395) (end -18.475 -10.2321) (width 0.762) (layer "F.Cu") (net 8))
 (segment (start -18.475 -3.953) (end -18.475 -2.1316) (width 0.762) (layer "F.Cu") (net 8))
 (segment (start -13.668001 -2.000001) (end -13.6779 -2.0099) (width 0.762) (layer "F.Cu") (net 8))
 (via (at -18.475 -3.953) (size 0.762) (drill 0.3048) (layers "F.Cu" "B.Cu") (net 8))
 (via (at -13.6779 -2.0099) (size 0.762) (drill 0.3048) (layers "F.Cu" "B.Cu") (free) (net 8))
 (segment (start -2.9337 -2.0607) (end -2.9337 -8.9187) (width 0.508) (layer "B.Cu") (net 8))
 (segment (start -16.5319 -2.0099) (end -13.6779 -2.0099) (width 0.508) (layer "B.Cu") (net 8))
 (segment (start -18.475 -3.953) (end -16.5319 -2.0099) (width 0.508) (layer "B.Cu") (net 8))
 (segment (start 2.2352 -14.0241) (end 9.1012 -14.0241) (width 0.508) (layer "B.Cu") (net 8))
 (segment (start -12.7508 -1.0828) (end -3.9116 -1.0828) (width 0.508) (layer "B.Cu") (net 8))
 (segment (start -3.9116 -1.0828) (end -2.9337 -2.0607) (width 0.508) (layer "B.Cu") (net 8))
 (segment (start -13.6779 -2.0099) (end -12.7508 -1.0828) (width 0.508) (layer "B.Cu") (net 8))
 (segment (start 9.1012 -14.0241) (end 10.3378 -15.2607) (width 0.508) (layer "B.Cu") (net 8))
 (segment (start -2.9337 -8.9187) (end 1.3335 -13.1859) (width 0.508) (layer "B.Cu") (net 8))
 (segment (start 1.3335 -13.1859) (end 1.397 -13.1859) (width 0.508) (layer "B.Cu") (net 8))
 (segment (start 1.397 -13.1859) (end 2.2352 -14.0241) (width 0.508) (layer "B.Cu") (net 8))
 (segment (start -9.525 -2.000001) (end -5.5 -2.000001) (width 0.508) (layer "F.Cu") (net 11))
 (segment (start -9.525 -2.000001) (end -5.5 -2.000001) (width 0.508) (layer "F.Cu") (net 11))
 (segment (start 1.475 -23.000001) (end 5.5 -23.000001) (width 0.508) (layer "F.Cu") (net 6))
 (segment (start 1.475 -20.200001) (end 5.5 -20.200001) (width 0.508) (layer "F.Cu") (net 15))
 (segment (start 1.475 -17.400001) (end 5.5 -17.400001) (width 0.508) (layer "F.Cu") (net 5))
 (segment (start 1.475 -14.600001) (end 5.5 -14.600001) (width 0.508) (layer "F.Cu") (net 10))
 (segment (start 1.475 -11.800001) (end 5.5 -11.800001) (width 0.508) (layer "F.Cu") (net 2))
 (segment (start 1.475 -9.000001) (end 5.5 -9.000001) (width 0.508) (layer "F.Cu") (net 1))
 (segment (start 1.475 -6.200001) (end 5.5 -6.200001) (width 0.508) (layer "F.Cu") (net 20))
 (segment (start 1.475 -3.400001) (end 5.5 -3.400001) (width 0.508) (layer "F.Cu") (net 4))
 (segment (start 9.309101 -0.700001) (end 10.3759 -1.7668) (width 0.508) (layer "F.Cu") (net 14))
 (segment (start 5.5 -0.700001) (end 9.309101 -0.700001) (width 0.508) (layer "F.Cu") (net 14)))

